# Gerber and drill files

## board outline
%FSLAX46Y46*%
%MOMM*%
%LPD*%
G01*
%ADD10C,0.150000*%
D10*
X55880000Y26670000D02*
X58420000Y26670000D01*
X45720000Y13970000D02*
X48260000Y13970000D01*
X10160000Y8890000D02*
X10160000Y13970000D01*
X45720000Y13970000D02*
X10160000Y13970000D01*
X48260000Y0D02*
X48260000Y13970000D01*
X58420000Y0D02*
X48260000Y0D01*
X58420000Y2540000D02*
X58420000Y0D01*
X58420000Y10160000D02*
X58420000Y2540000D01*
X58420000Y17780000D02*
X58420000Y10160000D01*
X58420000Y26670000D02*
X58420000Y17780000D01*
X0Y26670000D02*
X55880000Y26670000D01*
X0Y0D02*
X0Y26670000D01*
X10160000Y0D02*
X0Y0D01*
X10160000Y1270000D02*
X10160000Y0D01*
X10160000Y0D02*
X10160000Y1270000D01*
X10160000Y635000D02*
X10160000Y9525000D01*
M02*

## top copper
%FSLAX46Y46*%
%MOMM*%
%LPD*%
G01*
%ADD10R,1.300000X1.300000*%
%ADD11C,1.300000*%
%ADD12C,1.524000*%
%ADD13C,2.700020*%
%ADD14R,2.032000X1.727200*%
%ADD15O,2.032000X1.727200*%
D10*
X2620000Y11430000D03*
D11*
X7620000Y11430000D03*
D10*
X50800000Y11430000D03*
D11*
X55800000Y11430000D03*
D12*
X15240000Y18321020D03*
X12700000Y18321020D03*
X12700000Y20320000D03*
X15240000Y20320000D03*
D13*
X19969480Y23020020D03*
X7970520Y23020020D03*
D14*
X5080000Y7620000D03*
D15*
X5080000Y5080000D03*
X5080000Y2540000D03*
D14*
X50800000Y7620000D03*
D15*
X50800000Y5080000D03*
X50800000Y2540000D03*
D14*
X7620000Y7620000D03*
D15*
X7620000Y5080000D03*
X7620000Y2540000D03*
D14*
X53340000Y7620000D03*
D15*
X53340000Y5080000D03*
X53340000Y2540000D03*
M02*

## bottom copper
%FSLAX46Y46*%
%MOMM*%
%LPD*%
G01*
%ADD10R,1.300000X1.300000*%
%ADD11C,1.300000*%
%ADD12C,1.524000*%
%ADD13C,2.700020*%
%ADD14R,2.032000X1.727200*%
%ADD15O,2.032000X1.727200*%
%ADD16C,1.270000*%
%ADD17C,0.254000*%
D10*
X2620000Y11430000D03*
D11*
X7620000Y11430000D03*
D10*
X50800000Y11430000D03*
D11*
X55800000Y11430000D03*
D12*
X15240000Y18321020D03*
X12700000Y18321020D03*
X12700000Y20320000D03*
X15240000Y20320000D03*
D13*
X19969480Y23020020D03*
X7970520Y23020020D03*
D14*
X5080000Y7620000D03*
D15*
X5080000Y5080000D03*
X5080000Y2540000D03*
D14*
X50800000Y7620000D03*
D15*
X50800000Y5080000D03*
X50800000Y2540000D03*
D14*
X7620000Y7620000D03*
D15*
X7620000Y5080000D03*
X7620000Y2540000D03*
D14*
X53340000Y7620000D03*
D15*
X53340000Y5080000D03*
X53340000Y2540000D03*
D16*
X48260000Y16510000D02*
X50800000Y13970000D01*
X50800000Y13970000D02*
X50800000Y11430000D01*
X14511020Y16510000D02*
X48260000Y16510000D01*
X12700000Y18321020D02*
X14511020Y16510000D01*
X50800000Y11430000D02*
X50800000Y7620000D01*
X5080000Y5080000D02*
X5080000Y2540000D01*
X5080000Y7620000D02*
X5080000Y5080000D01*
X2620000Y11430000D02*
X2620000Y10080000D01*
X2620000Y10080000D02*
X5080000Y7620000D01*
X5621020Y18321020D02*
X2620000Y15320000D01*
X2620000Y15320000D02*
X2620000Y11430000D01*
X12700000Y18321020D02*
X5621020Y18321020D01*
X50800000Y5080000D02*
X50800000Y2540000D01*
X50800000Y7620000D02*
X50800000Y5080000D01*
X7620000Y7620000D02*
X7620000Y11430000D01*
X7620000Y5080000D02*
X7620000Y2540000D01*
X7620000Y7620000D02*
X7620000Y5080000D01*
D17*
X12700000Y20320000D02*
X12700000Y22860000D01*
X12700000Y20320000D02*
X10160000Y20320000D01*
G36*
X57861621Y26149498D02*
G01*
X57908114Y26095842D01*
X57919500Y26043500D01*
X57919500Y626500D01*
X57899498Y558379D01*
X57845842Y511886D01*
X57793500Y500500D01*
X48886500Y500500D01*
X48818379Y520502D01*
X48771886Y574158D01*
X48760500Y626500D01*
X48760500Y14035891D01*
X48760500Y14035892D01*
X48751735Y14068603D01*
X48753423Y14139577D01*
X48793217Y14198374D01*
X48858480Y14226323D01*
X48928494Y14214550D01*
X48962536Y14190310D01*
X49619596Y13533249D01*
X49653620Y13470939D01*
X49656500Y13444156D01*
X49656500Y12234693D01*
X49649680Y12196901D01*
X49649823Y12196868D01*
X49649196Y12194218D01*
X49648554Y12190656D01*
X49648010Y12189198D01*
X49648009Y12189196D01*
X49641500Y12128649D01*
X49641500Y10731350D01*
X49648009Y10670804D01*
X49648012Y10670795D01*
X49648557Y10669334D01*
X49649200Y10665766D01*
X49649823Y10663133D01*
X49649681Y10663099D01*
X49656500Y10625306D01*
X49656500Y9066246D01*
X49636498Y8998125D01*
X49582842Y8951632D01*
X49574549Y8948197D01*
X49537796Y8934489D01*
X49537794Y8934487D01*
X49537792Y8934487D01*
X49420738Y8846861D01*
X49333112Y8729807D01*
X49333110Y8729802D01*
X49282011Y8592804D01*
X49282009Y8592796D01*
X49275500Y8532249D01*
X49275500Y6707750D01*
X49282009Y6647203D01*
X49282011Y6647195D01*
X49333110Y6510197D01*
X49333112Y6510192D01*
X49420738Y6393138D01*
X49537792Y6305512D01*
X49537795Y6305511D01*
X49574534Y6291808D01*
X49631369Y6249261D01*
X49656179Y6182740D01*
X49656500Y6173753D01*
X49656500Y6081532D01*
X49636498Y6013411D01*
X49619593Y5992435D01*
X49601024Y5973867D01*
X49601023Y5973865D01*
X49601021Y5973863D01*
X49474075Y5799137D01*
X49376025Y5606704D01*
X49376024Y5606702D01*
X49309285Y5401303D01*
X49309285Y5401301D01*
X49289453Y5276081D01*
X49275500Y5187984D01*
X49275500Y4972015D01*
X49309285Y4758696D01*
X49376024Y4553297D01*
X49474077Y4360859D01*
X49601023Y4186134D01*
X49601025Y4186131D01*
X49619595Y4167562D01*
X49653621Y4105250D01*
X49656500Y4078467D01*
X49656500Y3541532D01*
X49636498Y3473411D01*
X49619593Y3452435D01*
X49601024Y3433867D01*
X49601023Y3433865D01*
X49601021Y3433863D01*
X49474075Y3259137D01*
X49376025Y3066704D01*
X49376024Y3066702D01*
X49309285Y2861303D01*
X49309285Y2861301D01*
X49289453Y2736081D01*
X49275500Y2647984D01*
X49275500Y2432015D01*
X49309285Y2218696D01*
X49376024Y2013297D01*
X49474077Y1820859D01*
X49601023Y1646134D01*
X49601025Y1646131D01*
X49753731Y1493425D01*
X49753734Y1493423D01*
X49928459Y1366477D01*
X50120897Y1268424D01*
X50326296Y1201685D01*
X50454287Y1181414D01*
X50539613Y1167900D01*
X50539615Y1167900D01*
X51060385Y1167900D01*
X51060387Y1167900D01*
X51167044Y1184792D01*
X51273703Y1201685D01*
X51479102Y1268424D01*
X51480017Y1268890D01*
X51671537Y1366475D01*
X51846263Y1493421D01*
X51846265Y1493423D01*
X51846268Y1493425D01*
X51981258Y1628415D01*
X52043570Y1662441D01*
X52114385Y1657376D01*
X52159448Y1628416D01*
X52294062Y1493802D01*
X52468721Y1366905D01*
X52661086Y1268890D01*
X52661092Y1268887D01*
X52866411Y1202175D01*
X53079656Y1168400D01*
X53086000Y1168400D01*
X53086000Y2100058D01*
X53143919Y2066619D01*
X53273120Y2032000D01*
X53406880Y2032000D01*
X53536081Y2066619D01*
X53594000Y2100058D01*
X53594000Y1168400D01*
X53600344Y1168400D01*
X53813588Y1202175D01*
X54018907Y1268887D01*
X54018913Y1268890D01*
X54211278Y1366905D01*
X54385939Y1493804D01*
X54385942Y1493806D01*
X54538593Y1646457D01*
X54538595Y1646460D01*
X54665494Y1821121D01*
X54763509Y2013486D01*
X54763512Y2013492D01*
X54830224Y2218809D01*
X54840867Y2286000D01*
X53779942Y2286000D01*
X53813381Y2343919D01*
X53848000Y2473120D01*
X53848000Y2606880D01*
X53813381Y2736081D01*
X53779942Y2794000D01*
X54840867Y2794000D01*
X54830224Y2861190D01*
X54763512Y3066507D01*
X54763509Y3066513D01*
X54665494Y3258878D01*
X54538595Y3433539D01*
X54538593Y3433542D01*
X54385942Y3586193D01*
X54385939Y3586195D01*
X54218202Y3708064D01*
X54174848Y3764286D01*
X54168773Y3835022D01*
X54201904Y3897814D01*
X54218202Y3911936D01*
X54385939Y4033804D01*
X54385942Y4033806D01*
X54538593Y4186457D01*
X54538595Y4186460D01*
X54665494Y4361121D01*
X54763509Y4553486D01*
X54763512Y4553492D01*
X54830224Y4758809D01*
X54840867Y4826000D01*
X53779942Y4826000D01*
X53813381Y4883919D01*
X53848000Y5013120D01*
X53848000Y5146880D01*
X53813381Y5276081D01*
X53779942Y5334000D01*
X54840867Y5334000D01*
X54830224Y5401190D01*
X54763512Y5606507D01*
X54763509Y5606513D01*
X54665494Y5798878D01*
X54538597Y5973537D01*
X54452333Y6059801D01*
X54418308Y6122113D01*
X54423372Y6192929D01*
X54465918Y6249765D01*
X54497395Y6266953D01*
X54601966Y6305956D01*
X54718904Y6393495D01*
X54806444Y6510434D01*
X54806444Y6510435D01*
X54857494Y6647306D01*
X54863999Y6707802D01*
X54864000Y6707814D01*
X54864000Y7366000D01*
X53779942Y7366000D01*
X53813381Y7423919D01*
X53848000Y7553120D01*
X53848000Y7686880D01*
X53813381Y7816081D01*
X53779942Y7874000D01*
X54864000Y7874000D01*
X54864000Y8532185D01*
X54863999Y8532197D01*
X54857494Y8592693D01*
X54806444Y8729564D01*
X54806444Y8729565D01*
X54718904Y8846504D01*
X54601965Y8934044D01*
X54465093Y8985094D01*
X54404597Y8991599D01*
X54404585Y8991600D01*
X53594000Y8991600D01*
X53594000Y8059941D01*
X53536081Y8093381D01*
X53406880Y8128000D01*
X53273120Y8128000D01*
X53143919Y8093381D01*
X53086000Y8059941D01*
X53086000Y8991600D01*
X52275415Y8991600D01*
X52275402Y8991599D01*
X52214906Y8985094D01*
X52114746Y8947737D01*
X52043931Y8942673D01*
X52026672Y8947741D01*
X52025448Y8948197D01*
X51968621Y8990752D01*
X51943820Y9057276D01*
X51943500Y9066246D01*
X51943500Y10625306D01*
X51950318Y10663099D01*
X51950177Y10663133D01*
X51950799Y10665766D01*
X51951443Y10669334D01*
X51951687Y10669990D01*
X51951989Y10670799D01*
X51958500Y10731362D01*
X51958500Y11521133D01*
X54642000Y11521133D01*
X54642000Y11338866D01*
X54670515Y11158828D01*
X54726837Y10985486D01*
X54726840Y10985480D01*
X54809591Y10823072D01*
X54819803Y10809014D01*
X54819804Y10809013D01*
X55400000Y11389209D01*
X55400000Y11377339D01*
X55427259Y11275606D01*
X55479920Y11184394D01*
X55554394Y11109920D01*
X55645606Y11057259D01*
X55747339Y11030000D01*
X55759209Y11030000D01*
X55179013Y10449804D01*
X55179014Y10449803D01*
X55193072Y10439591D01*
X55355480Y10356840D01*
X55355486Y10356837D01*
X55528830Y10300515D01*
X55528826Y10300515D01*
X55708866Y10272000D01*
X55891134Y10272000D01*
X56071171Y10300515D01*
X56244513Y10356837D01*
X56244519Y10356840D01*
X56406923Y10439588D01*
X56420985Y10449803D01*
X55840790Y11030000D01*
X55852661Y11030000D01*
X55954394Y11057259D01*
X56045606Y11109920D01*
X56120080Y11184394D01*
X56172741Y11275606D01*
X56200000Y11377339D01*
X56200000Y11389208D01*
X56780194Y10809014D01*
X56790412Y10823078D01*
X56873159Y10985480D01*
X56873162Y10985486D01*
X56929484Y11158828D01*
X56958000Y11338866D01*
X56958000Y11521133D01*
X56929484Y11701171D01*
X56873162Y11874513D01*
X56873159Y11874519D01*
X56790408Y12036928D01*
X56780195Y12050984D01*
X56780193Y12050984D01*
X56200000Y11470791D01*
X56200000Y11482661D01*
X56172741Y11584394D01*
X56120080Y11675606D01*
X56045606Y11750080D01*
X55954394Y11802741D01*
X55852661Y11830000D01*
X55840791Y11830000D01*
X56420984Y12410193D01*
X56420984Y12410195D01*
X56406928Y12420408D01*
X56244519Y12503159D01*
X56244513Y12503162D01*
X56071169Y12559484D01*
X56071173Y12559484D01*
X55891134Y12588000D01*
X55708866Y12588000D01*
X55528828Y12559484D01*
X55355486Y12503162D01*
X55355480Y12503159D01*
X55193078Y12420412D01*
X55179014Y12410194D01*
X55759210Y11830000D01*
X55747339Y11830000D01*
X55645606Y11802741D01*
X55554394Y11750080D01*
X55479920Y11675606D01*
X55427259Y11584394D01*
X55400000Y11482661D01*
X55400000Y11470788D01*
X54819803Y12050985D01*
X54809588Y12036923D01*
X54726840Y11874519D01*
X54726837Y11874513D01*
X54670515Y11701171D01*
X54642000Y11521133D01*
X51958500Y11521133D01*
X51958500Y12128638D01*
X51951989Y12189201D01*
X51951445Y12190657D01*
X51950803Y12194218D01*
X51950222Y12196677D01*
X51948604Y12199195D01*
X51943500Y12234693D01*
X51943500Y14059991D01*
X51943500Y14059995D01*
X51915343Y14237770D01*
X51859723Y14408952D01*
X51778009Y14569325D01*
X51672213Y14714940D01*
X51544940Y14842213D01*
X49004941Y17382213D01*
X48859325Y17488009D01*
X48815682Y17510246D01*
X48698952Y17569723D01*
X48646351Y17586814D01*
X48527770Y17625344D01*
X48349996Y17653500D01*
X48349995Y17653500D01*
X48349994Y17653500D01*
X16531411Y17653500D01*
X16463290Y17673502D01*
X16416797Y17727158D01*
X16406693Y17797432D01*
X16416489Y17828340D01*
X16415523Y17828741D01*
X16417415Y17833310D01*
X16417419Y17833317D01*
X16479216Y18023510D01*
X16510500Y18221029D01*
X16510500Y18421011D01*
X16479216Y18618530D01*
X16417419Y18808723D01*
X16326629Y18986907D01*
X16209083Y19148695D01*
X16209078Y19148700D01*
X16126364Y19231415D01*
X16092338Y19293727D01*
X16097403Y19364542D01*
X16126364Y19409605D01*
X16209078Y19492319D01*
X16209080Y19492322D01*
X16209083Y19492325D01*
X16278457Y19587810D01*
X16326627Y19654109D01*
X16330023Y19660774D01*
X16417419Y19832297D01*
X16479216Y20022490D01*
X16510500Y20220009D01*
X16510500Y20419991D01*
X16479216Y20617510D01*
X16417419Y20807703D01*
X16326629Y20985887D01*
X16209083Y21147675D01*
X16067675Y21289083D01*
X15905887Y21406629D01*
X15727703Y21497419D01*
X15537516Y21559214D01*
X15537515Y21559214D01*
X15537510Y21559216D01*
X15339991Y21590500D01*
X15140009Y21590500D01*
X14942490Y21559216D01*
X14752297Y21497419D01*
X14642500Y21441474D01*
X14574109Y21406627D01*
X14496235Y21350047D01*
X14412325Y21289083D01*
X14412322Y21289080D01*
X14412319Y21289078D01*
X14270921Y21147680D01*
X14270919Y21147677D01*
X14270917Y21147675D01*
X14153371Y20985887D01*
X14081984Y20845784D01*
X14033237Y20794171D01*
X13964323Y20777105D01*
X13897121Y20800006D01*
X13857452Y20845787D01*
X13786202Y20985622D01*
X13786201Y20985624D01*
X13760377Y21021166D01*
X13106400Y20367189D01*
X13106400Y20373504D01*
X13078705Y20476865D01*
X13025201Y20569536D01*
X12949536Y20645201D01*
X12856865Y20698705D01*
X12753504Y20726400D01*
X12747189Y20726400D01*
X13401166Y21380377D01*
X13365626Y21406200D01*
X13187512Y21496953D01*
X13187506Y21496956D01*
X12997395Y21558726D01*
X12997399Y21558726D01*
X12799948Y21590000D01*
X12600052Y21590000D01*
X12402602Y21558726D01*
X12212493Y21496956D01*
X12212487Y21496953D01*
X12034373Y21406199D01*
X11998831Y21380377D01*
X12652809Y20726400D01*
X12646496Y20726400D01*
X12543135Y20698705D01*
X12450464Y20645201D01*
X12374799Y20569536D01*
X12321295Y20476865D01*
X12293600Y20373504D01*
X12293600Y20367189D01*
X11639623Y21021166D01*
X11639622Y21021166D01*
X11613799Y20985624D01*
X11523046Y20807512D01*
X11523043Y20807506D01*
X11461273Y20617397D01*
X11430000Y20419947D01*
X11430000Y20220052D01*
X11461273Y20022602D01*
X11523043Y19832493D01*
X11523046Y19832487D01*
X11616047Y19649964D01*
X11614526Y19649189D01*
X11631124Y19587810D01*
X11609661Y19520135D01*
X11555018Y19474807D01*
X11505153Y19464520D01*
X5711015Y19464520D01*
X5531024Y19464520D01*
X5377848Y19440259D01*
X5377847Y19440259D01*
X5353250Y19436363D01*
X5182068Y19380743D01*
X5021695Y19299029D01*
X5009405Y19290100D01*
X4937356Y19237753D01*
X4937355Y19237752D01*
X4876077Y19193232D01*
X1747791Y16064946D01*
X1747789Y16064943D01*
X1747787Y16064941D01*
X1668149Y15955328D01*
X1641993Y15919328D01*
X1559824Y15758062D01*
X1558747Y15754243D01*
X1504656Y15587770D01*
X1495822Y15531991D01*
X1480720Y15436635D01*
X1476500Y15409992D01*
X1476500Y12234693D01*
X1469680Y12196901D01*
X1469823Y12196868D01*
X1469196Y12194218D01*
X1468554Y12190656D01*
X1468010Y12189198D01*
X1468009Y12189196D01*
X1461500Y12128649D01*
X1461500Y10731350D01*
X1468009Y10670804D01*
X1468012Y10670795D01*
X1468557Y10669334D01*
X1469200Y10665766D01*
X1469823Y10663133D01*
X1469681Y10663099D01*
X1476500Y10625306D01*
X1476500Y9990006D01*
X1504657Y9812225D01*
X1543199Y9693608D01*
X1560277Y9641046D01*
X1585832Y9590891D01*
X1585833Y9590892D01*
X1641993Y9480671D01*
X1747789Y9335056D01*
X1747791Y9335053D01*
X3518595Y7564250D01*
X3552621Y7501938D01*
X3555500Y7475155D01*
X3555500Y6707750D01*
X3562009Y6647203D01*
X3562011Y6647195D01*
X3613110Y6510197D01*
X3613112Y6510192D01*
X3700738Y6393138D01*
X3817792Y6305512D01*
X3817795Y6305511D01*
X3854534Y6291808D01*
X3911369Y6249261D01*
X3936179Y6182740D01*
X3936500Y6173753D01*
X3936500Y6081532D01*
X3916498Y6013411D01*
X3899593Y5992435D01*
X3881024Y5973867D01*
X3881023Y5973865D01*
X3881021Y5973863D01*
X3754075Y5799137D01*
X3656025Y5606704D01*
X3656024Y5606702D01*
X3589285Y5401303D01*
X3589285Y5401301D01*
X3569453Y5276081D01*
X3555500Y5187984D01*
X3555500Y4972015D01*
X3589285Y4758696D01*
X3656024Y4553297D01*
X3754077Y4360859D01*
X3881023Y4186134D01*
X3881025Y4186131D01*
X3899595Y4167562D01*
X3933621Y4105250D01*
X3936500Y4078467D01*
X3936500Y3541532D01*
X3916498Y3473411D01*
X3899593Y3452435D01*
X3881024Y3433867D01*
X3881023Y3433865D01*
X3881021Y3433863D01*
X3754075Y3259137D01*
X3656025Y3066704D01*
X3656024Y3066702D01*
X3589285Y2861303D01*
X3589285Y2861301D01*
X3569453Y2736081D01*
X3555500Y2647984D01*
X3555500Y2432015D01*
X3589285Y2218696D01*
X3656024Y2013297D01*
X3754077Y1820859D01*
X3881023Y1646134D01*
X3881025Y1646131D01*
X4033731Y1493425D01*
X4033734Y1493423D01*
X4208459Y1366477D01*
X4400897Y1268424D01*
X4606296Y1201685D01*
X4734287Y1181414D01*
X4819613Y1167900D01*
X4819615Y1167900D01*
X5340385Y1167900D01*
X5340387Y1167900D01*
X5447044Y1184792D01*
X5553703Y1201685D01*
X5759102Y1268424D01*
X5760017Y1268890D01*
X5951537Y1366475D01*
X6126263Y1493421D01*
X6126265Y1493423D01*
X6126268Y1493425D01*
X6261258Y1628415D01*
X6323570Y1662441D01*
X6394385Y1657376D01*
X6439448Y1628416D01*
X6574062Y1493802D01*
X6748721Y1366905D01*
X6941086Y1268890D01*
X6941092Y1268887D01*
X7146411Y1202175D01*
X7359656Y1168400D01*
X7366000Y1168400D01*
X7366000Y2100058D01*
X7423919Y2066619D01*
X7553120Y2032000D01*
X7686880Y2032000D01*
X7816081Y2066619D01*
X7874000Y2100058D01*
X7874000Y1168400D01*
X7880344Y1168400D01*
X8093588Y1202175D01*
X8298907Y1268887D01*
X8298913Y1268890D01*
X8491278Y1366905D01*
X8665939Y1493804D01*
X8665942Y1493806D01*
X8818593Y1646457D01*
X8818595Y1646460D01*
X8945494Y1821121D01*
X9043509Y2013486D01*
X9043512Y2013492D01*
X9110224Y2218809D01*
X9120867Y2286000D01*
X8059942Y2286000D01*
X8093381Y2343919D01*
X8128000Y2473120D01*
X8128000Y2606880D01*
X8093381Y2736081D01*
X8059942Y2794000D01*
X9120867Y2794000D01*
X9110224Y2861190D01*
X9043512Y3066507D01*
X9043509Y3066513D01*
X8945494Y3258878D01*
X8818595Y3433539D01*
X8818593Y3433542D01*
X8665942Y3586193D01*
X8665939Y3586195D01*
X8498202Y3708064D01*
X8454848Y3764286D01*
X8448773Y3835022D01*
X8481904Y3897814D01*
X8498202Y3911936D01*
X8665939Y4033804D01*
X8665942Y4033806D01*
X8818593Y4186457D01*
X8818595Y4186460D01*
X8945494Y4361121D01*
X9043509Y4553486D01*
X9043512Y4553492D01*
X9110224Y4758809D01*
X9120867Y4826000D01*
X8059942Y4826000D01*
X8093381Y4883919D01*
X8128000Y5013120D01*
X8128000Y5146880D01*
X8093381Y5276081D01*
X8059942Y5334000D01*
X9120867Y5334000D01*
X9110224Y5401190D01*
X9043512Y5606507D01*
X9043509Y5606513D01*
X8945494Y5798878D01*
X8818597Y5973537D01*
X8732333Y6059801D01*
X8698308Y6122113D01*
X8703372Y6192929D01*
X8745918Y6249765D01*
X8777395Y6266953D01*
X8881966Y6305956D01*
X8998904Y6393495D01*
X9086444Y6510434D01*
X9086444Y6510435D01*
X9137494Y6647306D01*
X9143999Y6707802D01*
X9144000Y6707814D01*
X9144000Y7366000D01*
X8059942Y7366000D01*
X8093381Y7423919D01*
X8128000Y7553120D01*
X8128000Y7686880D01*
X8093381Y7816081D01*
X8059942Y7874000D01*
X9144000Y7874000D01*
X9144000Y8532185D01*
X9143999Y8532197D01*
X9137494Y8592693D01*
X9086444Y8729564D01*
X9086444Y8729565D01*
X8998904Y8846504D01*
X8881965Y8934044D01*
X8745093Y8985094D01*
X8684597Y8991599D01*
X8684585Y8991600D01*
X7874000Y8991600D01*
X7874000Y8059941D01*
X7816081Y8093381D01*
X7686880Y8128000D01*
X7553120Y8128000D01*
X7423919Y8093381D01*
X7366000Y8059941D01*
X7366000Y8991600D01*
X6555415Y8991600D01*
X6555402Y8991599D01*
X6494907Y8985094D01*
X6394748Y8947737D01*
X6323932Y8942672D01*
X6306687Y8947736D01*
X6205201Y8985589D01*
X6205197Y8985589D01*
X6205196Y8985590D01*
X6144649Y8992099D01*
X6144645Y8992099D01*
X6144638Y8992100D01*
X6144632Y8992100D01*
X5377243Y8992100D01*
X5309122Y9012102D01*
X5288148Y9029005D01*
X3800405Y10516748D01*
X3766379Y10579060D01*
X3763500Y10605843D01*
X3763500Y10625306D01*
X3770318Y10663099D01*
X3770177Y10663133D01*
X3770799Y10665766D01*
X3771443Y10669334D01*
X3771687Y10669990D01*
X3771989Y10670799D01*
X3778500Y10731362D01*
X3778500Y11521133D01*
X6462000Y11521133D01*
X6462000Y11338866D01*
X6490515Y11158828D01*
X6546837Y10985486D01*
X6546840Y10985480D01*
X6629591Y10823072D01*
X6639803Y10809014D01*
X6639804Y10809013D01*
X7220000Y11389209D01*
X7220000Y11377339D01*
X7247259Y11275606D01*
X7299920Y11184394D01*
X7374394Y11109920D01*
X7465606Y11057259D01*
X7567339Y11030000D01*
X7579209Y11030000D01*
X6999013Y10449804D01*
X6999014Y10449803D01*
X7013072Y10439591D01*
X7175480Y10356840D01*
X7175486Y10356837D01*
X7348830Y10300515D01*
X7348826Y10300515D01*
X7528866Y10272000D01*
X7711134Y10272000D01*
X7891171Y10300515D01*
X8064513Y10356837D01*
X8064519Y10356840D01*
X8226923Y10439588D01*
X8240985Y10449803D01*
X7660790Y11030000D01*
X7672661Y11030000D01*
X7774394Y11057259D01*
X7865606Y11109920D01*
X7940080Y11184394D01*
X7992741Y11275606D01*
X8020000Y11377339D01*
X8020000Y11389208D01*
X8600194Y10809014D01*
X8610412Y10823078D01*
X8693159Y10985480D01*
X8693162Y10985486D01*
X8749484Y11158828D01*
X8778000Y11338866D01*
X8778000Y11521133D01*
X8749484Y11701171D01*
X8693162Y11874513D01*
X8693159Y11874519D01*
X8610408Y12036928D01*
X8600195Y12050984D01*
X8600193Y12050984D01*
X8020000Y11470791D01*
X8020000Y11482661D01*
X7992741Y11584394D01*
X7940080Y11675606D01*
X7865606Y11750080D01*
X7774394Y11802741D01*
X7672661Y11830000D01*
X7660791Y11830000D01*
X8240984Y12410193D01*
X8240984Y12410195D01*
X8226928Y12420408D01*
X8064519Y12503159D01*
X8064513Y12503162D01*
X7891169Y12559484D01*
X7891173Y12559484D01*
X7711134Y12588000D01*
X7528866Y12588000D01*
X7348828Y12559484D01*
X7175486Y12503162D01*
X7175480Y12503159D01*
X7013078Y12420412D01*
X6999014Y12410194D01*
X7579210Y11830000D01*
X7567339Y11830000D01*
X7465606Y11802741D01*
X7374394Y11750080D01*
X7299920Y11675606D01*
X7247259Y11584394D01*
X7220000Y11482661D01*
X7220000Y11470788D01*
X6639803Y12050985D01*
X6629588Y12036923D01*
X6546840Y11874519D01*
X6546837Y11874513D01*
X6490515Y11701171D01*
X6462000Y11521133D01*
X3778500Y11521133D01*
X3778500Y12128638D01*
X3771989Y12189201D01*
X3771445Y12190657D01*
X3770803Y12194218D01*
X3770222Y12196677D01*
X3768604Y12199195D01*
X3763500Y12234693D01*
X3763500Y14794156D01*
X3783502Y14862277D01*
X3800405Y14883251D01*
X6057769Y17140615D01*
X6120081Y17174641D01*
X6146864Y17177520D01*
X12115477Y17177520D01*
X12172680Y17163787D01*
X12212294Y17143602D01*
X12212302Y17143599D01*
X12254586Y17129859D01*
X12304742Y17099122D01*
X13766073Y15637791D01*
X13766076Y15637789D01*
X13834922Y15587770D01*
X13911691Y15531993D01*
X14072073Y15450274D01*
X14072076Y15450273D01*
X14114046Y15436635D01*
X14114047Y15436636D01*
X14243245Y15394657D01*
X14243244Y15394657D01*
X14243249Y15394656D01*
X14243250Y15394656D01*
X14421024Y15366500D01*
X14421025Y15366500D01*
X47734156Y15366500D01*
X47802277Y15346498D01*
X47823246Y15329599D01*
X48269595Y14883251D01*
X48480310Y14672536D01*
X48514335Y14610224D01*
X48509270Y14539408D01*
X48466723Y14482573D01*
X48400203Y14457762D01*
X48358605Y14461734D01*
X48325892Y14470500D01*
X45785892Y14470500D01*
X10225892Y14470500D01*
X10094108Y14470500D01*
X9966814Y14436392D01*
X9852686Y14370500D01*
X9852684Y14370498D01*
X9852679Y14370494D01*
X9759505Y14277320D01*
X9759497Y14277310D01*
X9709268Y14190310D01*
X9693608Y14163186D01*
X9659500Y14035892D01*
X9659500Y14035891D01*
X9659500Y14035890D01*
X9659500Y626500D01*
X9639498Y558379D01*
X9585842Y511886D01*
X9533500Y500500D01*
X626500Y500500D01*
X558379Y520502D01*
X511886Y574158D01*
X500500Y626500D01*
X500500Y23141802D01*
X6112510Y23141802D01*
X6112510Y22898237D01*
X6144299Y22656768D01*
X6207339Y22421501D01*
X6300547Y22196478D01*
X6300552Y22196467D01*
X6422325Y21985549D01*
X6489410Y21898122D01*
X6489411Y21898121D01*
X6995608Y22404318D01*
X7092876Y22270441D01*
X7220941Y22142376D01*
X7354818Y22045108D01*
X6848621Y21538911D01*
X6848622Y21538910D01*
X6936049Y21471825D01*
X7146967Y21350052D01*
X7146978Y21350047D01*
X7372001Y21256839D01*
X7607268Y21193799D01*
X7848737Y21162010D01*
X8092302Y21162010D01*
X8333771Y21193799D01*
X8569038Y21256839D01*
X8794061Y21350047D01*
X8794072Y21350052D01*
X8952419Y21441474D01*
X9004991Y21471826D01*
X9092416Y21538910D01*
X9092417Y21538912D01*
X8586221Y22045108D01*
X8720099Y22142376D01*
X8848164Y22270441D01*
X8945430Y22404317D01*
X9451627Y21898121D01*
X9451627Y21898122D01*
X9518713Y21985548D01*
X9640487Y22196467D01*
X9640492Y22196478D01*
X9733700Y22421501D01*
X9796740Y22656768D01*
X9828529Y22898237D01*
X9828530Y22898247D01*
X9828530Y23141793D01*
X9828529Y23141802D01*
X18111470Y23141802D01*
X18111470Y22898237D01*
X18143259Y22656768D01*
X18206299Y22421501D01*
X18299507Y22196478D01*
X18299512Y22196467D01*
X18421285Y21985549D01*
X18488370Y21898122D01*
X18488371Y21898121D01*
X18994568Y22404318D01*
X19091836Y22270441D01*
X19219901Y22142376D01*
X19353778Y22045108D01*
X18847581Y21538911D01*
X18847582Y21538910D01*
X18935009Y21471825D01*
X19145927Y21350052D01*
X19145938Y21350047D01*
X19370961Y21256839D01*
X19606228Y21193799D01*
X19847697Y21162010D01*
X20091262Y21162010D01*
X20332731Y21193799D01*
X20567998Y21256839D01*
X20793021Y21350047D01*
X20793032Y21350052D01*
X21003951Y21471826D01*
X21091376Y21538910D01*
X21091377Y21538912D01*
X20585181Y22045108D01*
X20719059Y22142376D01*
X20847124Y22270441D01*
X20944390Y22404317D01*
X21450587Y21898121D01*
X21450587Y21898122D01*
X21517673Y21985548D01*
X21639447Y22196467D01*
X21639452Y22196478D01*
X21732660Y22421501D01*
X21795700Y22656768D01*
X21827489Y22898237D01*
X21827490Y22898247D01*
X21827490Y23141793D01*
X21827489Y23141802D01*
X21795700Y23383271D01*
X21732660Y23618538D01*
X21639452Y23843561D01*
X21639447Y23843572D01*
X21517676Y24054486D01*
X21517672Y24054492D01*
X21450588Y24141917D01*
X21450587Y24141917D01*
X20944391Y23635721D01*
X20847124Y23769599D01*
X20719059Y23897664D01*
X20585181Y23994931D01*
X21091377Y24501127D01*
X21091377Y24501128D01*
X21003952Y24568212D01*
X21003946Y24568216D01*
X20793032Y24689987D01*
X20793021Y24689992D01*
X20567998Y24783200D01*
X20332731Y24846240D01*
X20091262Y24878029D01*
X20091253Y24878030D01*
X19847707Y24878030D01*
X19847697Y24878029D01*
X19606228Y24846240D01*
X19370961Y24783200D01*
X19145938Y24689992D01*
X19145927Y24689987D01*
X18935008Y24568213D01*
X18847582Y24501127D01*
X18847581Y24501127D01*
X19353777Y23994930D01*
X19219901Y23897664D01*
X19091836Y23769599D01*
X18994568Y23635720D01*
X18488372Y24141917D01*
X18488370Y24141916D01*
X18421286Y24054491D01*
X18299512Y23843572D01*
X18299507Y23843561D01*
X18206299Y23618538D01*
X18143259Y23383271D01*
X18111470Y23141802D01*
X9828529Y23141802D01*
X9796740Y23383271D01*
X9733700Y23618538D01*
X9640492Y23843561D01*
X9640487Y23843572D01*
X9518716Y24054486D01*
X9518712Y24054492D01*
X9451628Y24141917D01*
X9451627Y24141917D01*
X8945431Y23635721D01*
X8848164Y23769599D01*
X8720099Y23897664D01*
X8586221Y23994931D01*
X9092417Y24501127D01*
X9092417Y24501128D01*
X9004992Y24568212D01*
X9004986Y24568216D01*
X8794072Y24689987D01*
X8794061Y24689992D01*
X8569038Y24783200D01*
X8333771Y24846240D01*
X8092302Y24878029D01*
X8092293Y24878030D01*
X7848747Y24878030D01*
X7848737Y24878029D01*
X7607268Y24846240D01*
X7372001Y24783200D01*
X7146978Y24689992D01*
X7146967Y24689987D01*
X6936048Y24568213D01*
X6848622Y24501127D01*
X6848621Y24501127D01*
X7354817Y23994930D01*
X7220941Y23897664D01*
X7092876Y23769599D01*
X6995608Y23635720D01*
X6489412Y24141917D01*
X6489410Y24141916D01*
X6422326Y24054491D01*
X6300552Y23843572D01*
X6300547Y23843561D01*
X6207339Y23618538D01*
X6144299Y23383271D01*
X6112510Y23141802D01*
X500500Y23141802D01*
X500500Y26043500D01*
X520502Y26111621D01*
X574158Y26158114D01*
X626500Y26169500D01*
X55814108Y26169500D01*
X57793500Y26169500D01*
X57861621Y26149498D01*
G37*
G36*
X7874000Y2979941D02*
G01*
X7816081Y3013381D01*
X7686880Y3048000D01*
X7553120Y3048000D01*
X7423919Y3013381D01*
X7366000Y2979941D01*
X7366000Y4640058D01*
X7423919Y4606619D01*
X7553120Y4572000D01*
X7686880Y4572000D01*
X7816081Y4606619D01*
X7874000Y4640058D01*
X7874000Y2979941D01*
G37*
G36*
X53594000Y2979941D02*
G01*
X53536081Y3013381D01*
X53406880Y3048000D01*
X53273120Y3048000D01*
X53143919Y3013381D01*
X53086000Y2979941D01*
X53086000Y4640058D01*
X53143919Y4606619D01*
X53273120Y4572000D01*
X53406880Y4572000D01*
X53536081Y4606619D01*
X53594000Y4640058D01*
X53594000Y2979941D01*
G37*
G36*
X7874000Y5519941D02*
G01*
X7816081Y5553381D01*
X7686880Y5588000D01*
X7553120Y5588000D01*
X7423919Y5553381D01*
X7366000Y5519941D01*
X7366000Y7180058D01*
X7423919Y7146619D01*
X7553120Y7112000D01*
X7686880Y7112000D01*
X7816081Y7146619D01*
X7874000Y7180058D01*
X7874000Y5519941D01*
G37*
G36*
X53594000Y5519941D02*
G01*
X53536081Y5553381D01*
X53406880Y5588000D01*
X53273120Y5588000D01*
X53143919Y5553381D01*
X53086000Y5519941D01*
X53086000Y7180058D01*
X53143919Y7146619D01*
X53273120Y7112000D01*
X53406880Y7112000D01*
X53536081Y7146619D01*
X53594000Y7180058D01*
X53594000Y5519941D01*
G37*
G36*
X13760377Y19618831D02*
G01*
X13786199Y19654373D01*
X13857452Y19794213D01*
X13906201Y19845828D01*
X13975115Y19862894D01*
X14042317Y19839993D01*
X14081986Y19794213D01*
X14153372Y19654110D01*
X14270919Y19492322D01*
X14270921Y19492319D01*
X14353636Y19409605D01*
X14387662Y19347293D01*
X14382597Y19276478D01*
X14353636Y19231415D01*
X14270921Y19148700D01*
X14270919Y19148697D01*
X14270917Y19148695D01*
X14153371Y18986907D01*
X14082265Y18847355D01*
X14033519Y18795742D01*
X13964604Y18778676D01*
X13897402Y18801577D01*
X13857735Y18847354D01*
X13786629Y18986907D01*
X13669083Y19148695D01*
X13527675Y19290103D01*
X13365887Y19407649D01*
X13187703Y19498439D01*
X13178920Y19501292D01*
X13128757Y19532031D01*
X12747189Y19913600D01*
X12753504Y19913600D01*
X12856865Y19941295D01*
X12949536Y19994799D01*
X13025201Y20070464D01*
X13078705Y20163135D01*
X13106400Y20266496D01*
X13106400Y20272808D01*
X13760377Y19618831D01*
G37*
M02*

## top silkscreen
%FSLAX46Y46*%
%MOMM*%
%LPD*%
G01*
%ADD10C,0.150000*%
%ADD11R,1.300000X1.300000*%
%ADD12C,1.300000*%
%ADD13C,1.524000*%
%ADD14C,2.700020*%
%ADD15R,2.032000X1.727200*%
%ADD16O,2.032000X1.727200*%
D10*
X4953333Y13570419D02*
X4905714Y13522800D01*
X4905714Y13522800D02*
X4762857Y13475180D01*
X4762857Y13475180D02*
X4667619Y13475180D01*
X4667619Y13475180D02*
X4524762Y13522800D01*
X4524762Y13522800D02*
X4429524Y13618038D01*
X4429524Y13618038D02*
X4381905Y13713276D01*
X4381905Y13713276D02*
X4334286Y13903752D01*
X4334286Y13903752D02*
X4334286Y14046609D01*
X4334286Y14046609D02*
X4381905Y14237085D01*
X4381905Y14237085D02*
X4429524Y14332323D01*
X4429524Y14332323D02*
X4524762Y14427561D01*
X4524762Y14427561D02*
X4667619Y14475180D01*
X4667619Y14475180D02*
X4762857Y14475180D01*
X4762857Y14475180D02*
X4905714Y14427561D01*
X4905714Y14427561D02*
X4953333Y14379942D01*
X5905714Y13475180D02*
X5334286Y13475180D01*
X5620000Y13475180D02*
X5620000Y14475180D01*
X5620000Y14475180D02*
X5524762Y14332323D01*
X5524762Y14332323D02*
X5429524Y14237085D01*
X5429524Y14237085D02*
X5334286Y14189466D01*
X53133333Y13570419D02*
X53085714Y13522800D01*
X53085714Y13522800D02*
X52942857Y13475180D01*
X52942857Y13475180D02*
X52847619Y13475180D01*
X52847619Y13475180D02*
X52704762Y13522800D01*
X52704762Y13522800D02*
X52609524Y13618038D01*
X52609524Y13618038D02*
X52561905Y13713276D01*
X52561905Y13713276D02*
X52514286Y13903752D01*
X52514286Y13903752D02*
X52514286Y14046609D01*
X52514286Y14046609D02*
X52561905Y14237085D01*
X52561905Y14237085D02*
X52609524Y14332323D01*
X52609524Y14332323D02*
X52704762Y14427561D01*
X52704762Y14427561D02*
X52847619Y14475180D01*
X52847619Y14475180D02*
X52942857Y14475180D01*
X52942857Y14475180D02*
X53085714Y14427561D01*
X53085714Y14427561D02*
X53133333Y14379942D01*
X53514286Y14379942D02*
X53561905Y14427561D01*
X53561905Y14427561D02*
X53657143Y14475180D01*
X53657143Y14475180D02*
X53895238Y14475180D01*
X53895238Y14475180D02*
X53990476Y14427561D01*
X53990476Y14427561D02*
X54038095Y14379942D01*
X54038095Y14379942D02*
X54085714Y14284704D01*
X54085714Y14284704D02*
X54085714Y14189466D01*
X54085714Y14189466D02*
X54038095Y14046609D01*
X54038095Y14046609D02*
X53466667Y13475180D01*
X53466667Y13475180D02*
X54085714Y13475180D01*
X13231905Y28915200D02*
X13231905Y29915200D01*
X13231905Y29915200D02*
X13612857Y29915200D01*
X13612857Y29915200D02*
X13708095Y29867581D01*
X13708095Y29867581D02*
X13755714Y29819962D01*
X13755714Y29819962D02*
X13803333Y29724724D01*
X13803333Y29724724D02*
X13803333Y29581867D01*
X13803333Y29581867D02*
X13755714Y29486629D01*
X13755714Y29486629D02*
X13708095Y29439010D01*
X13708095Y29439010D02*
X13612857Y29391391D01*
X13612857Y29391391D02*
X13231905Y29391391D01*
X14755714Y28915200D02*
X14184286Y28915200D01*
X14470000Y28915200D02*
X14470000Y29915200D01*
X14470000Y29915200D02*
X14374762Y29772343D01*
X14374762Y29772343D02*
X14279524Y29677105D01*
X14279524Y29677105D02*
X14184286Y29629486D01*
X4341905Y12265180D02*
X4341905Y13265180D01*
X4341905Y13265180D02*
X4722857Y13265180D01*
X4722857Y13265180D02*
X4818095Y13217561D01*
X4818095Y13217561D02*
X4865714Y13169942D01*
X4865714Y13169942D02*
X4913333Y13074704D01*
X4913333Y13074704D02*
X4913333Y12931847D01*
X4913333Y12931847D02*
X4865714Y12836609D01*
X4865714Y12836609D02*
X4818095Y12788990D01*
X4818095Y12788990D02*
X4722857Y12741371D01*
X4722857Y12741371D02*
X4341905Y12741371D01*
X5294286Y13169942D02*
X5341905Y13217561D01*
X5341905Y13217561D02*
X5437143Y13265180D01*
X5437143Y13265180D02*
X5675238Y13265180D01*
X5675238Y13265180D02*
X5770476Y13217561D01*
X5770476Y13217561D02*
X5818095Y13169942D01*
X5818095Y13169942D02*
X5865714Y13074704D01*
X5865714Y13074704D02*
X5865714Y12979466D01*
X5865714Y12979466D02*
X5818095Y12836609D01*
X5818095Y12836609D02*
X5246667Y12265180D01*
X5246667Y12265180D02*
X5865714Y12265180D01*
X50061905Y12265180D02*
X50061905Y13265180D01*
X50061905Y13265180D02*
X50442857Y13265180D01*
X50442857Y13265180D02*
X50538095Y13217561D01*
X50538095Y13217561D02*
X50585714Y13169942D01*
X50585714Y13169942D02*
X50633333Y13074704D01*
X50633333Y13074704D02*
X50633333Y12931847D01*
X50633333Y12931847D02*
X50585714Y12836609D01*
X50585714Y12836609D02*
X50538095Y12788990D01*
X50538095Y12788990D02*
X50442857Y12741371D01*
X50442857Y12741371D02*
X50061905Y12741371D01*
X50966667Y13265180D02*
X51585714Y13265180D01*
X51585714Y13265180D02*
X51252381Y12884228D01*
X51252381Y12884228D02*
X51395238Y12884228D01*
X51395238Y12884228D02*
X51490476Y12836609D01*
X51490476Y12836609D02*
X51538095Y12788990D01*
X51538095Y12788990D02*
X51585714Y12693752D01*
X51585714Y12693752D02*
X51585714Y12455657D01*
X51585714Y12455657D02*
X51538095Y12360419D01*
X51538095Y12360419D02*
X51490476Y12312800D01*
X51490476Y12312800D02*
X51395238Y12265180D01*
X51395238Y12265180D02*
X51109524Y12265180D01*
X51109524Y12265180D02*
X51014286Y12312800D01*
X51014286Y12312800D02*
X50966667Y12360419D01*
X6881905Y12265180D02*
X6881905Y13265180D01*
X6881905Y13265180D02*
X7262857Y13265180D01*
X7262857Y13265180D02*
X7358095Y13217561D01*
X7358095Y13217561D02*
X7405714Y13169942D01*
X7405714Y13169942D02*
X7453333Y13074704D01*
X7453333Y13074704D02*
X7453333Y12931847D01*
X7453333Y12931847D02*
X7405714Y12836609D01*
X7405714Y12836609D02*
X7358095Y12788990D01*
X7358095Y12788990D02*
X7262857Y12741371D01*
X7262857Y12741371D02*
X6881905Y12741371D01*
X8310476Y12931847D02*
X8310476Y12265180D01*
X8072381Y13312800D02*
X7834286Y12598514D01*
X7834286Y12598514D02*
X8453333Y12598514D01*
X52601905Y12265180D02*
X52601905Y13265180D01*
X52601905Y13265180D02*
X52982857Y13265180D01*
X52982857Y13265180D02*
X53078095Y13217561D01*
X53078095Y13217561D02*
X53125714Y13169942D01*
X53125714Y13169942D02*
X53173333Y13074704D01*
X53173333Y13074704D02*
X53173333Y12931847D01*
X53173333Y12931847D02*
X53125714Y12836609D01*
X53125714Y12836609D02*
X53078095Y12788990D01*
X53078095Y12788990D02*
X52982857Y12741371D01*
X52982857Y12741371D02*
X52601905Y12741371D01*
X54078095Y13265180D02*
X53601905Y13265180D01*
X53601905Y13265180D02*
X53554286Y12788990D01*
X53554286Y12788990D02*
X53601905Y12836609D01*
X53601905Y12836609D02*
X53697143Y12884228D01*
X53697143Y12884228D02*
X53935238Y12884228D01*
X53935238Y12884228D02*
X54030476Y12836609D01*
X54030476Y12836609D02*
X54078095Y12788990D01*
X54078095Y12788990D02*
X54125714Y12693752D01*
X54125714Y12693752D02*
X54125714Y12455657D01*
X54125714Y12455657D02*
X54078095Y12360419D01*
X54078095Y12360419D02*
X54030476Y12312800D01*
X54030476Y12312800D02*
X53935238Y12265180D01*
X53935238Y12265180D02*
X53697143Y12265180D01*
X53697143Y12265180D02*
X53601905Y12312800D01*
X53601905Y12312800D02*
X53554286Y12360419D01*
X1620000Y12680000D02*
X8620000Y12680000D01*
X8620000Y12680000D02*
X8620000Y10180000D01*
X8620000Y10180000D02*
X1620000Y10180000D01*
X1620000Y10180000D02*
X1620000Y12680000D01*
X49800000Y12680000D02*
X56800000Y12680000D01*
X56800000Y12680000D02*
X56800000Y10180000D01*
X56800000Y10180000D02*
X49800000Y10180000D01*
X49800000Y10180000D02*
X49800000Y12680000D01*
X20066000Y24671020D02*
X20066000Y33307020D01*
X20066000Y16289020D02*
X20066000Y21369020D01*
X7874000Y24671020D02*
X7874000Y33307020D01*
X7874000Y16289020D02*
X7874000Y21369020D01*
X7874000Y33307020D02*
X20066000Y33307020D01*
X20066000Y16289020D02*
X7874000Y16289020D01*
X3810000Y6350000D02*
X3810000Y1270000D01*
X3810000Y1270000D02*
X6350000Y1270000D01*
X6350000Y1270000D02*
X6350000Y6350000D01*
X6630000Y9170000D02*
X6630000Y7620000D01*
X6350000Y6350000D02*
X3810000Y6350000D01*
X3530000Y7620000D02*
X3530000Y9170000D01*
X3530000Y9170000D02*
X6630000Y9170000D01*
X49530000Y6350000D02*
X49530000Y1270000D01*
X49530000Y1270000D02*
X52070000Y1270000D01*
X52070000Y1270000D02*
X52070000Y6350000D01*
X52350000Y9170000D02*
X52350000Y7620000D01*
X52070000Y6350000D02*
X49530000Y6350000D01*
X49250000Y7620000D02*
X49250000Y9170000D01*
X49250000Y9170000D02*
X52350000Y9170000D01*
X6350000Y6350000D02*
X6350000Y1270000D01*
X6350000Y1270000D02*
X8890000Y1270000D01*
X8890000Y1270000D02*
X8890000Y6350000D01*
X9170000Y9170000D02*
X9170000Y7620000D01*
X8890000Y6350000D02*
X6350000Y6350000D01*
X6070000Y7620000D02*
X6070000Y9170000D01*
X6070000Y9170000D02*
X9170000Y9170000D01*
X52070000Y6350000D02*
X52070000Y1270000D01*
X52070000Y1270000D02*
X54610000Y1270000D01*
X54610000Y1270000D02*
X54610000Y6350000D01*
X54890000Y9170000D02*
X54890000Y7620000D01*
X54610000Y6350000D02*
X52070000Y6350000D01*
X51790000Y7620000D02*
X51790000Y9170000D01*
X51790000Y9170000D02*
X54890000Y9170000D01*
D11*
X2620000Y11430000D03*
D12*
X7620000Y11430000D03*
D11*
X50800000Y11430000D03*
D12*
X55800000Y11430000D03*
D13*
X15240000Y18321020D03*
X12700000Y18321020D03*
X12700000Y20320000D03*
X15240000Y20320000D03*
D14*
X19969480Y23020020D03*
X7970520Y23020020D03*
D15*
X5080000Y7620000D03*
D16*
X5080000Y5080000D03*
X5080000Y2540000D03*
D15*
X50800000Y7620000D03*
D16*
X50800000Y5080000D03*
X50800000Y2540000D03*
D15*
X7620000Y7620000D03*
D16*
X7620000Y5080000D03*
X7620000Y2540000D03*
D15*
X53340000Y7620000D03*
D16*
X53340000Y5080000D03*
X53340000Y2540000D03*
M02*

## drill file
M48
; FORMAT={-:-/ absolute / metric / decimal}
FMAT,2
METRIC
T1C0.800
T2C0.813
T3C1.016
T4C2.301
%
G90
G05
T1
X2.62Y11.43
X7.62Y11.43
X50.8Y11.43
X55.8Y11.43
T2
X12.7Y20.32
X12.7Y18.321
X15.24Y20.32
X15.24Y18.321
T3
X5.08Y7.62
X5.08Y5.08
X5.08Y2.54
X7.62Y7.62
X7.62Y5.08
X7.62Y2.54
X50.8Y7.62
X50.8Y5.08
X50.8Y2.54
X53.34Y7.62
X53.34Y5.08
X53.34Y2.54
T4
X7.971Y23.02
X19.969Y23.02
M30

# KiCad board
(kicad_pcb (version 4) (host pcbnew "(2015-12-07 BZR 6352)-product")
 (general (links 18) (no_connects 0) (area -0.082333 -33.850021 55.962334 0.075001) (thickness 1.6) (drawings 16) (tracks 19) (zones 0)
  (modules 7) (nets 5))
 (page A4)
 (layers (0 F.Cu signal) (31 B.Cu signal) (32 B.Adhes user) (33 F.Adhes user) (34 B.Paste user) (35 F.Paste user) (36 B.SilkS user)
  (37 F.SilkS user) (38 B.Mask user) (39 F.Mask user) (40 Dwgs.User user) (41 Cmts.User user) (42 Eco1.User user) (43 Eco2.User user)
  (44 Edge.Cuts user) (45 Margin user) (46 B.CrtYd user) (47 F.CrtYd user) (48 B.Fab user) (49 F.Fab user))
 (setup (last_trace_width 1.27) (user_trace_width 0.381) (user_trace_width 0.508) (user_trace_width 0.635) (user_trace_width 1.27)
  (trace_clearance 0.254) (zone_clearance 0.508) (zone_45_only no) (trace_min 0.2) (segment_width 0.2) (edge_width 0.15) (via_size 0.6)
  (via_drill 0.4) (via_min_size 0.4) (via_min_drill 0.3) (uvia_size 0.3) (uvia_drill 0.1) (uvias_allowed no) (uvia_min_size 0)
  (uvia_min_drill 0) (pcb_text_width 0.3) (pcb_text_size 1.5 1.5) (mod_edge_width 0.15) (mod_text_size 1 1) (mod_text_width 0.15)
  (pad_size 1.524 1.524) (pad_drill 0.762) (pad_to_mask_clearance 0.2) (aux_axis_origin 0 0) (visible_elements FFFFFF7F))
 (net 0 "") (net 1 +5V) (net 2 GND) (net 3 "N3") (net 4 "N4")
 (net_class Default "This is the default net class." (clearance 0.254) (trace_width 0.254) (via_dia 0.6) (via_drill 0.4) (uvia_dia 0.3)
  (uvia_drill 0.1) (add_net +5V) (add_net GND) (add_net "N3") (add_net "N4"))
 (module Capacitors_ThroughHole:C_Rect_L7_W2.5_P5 (layer F.Cu) (at 2.62 -11.43)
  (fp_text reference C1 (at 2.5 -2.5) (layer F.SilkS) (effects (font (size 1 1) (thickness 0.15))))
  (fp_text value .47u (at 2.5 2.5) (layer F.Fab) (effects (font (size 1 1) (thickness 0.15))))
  (fp_line (start -1 -1.25) (end 6 -1.25) (layer F.SilkS) (width 0.15))
  (fp_line (start 6 -1.25) (end 6 1.25) (layer F.SilkS) (width 0.15))
  (fp_line (start 6 1.25) (end -1 1.25) (layer F.SilkS) (width 0.15))
  (fp_line (start -1 1.25) (end -1 -1.25) (layer F.SilkS) (width 0.15))
  (pad 1 thru_hole rect (at 0 0) (size 1.3 1.3) (drill 0.8) (layers *.Cu *.Mask F.SilkS) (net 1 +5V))
  (pad 2 thru_hole circle (at 5 0) (size 1.3 1.3) (drill 0.8) (layers *.Cu *.Mask F.SilkS) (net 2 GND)))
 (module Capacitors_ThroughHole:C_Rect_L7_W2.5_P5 (layer F.Cu) (at 50.8 -11.43)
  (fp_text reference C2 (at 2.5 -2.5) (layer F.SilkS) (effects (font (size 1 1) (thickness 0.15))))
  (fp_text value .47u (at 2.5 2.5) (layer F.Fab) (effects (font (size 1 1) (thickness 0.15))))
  (fp_line (start -1 -1.25) (end 6 -1.25) (layer F.SilkS) (width 0.15))
  (fp_line (start 6 -1.25) (end 6 1.25) (layer F.SilkS) (width 0.15))
  (fp_line (start 6 1.25) (end -1 1.25) (layer F.SilkS) (width 0.15))
  (fp_line (start -1 1.25) (end -1 -1.25) (layer F.SilkS) (width 0.15))
  (pad 1 thru_hole rect (at 0 0) (size 1.3 1.3) (drill 0.8) (layers *.Cu *.Mask F.SilkS) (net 1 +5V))
  (pad 2 thru_hole circle (at 5 0) (size 1.3 1.3) (drill 0.8) (layers *.Cu *.Mask F.SilkS) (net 2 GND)))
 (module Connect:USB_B (layer F.Cu) (at 12.7 -18.32102 90)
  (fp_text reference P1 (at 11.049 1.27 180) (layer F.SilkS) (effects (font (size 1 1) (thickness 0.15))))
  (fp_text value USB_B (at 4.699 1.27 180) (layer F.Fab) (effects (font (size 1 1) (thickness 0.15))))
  (fp_line (start 6.35 7.366) (end 14.986 7.366) (layer F.SilkS) (width 0.15))
  (fp_line (start -2.032 7.366) (end 3.048 7.366) (layer F.SilkS) (width 0.15))
  (fp_line (start 6.35 -4.826) (end 14.986 -4.826) (layer F.SilkS) (width 0.15))
  (fp_line (start -2.032 -4.826) (end 3.048 -4.826) (layer F.SilkS) (width 0.15))
  (fp_line (start 14.986 -4.826) (end 14.986 7.366) (layer F.SilkS) (width 0.15))
  (fp_line (start -2.032 7.366) (end -2.032 -4.826) (layer F.SilkS) (width 0.15))
  (pad 2 thru_hole circle (at 0 2.54) (size 1.524 1.524) (drill 0.8128) (layers *.Cu *.Mask F.SilkS) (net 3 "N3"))
  (pad 1 thru_hole circle (at 0 0) (size 1.524 1.524) (drill 0.8128) (layers *.Cu *.Mask F.SilkS) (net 1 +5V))
  (pad 4 thru_hole circle (at 1.99898 0) (size 1.524 1.524) (drill 0.8128) (layers *.Cu *.Mask F.SilkS) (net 2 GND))
  (pad 3 thru_hole circle (at 1.99898 2.54) (size 1.524 1.524) (drill 0.8128) (layers *.Cu *.Mask F.SilkS) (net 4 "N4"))
  (pad 5 thru_hole circle (at 4.699 7.26948) (size 2.70002 2.70002) (drill 2.30124) (layers *.Cu *.Mask F.SilkS) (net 2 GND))
  (pad 5 thru_hole circle (at 4.699 -4.72948) (size 2.70002 2.70002) (drill 2.30124) (layers *.Cu *.Mask F.SilkS) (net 2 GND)))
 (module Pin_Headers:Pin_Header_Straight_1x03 (layer F.Cu) (at 5.08 -7.62)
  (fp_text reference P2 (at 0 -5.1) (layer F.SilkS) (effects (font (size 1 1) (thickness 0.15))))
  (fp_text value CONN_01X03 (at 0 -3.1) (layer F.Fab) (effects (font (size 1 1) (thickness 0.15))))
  (fp_line (start -1.27 1.27) (end -1.27 6.35) (layer F.SilkS) (width 0.15))
  (fp_line (start -1.27 6.35) (end 1.27 6.35) (layer F.SilkS) (width 0.15))
  (fp_line (start 1.27 6.35) (end 1.27 1.27) (layer F.SilkS) (width 0.15))
  (fp_line (start 1.55 -1.55) (end 1.55 0) (layer F.SilkS) (width 0.15))
  (fp_line (start 1.27 1.27) (end -1.27 1.27) (layer F.SilkS) (width 0.15))
  (fp_line (start -1.55 0) (end -1.55 -1.55) (layer F.SilkS) (width 0.15))
  (fp_line (start -1.55 -1.55) (end 1.55 -1.55) (layer F.SilkS) (width 0.15))
  (pad 1 thru_hole rect (at 0 0) (size 2.032 1.7272) (drill 1.016) (layers *.Cu *.Mask F.SilkS) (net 1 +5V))
  (pad 2 thru_hole oval (at 0 2.54) (size 2.032 1.7272) (drill 1.016) (layers *.Cu *.Mask F.SilkS) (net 1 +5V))
  (pad 3 thru_hole oval (at 0 5.08) (size 2.032 1.7272) (drill 1.016) (layers *.Cu *.Mask F.SilkS) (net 1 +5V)))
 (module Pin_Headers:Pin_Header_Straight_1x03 (layer F.Cu) (at 50.8 -7.62)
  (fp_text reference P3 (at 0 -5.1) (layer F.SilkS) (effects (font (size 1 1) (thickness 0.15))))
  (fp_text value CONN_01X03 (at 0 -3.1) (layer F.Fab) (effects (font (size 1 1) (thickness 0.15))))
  (fp_line (start -1.27 1.27) (end -1.27 6.35) (layer F.SilkS) (width 0.15))
  (fp_line (start -1.27 6.35) (end 1.27 6.35) (layer F.SilkS) (width 0.15))
  (fp_line (start 1.27 6.35) (end 1.27 1.27) (layer F.SilkS) (width 0.15))
  (fp_line (start 1.55 -1.55) (end 1.55 0) (layer F.SilkS) (width 0.15))
  (fp_line (start 1.27 1.27) (end -1.27 1.27) (layer F.SilkS) (width 0.15))
  (fp_line (start -1.55 0) (end -1.55 -1.55) (layer F.SilkS) (width 0.15))
  (fp_line (start -1.55 -1.55) (end 1.55 -1.55) (layer F.SilkS) (width 0.15))
  (pad 1 thru_hole rect (at 0 0) (size 2.032 1.7272) (drill 1.016) (layers *.Cu *.Mask F.SilkS) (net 1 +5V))
  (pad 2 thru_hole oval (at 0 2.54) (size 2.032 1.7272) (drill 1.016) (layers *.Cu *.Mask F.SilkS) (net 1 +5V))
  (pad 3 thru_hole oval (at 0 5.08) (size 2.032 1.7272) (drill 1.016) (layers *.Cu *.Mask F.SilkS) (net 1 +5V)))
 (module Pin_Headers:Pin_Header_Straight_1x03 (layer F.Cu) (at 7.62 -7.62)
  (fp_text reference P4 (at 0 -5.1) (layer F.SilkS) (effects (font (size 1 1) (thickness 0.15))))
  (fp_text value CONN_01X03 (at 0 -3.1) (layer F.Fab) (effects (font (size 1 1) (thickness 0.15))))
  (fp_line (start -1.27 1.27) (end -1.27 6.35) (layer F.SilkS) (width 0.15))
  (fp_line (start -1.27 6.35) (end 1.27 6.35) (layer F.SilkS) (width 0.15))
  (fp_line (start 1.27 6.35) (end 1.27 1.27) (layer F.SilkS) (width 0.15))
  (fp_line (start 1.55 -1.55) (end 1.55 0) (layer F.SilkS) (width 0.15))
  (fp_line (start 1.27 1.27) (end -1.27 1.27) (layer F.SilkS) (width 0.15))
  (fp_line (start -1.55 0) (end -1.55 -1.55) (layer F.SilkS) (width 0.15))
  (fp_line (start -1.55 -1.55) (end 1.55 -1.55) (layer F.SilkS) (width 0.15))
  (pad 1 thru_hole rect (at 0 0) (size 2.032 1.7272) (drill 1.016) (layers *.Cu *.Mask F.SilkS) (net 2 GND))
  (pad 2 thru_hole oval (at 0 2.54) (size 2.032 1.7272) (drill 1.016) (layers *.Cu *.Mask F.SilkS) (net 2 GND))
  (pad 3 thru_hole oval (at 0 5.08) (size 2.032 1.7272) (drill 1.016) (layers *.Cu *.Mask F.SilkS) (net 2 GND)))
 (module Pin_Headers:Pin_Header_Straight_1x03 (layer F.Cu) (at 53.34 -7.62)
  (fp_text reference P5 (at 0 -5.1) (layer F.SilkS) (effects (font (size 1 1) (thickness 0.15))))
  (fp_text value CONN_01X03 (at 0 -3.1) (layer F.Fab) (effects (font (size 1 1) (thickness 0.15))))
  (fp_line (start -1.27 1.27) (end -1.27 6.35) (layer F.SilkS) (width 0.15))
  (fp_line (start -1.27 6.35) (end 1.27 6.35) (layer F.SilkS) (width 0.15))
  (fp_line (start 1.27 6.35) (end 1.27 1.27) (layer F.SilkS) (width 0.15))
  (fp_line (start 1.55 -1.55) (end 1.55 0) (layer F.SilkS) (width 0.15))
  (fp_line (start 1.27 1.27) (end -1.27 1.27) (layer F.SilkS) (width 0.15))
  (fp_line (start -1.55 0) (end -1.55 -1.55) (layer F.SilkS) (width 0.15))
  (fp_line (start -1.55 -1.55) (end 1.55 -1.55) (layer F.SilkS) (width 0.15))
  (pad 1 thru_hole rect (at 0 0) (size 2.032 1.7272) (drill 1.016) (layers *.Cu *.Mask F.SilkS) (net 2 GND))
  (pad 2 thru_hole oval (at 0 2.54) (size 2.032 1.7272) (drill 1.016) (layers *.Cu *.Mask F.SilkS) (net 2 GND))
  (pad 3 thru_hole oval (at 0 5.08) (size 2.032 1.7272) (drill 1.016) (layers *.Cu *.Mask F.SilkS) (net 2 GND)))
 (gr_line (start 55.88 -26.67) (end 58.42 -26.67) (layer Edge.Cuts) (width 0.15))
 (gr_line (start 45.72 -13.97) (end 48.26 -13.97) (layer Edge.Cuts) (width 0.15))
 (gr_line (start 10.16 -8.89) (end 10.16 -13.97) (layer Edge.Cuts) (width 0.15))
 (gr_line (start 45.72 -13.97) (end 10.16 -13.97) (layer Edge.Cuts) (width 0.15))
 (gr_line (start 48.26 0) (end 48.26 -13.97) (layer Edge.Cuts) (width 0.15))
 (gr_line (start 58.42 0) (end 48.26 0) (layer Edge.Cuts) (width 0.15))
 (gr_line (start 58.42 -2.54) (end 58.42 0) (layer Edge.Cuts) (width 0.15))
 (gr_line (start 58.42 -10.16) (end 58.42 -2.54) (layer Edge.Cuts) (width 0.15))
 (gr_line (start 58.42 -17.78) (end 58.42 -10.16) (layer Edge.Cuts) (width 0.15))
 (gr_line (start 58.42 -26.67) (end 58.42 -17.78) (layer Edge.Cuts) (width 0.15))
 (gr_line (start 0 -26.67) (end 55.88 -26.67) (layer Edge.Cuts) (width 0.15))
 (gr_line (start 0 0) (end 0 -26.67) (layer Edge.Cuts) (width 0.15))
 (gr_line (start 10.16 0) (end 0 0) (layer Edge.Cuts) (width 0.15))
 (gr_line (start 10.16 -1.27) (end 10.16 0) (layer Edge.Cuts) (width 0.15))
 (gr_line (start 10.16 0) (end 10.16 -1.27) (layer Edge.Cuts) (width 0.15))
 (gr_line (start 10.16 -0.635) (end 10.16 -9.525) (layer Edge.Cuts) (width 0.15))
 (segment (start 48.26 -16.51) (end 50.8 -13.97) (width 1.27) (layer B.Cu) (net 1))
 (segment (start 50.8 -13.97) (end 50.8 -11.43) (width 1.27) (layer B.Cu) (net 1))
 (segment (start 14.51102 -16.51) (end 48.26 -16.51) (width 1.27) (layer B.Cu) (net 1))
 (segment (start 12.7 -18.32102) (end 14.51102 -16.51) (width 1.27) (layer B.Cu) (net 1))
 (segment (start 50.8 -11.43) (end 50.8 -7.62) (width 1.27) (layer B.Cu) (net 1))
 (segment (start 5.08 -5.08) (end 5.08 -2.54) (width 1.27) (layer B.Cu) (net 1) (status 30))
 (segment (start 5.08 -7.62) (end 5.08 -5.08) (width 1.27) (layer B.Cu) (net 1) (status 30))
 (segment (start 2.62 -11.43) (end 2.62 -10.08) (width 1.27) (layer B.Cu) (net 1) (status 10))
 (segment (start 2.62 -10.08) (end 5.08 -7.62) (width 1.27) (layer B.Cu) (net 1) (status 20))
 (segment (start 5.62102 -18.32102) (end 2.62 -15.32) (width 1.27) (layer B.Cu) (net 1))
 (segment (start 2.62 -15.32) (end 2.62 -11.43) (width 1.27) (layer B.Cu) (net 1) (status 20))
 (segment (start 12.7 -18.32102) (end 5.62102 -18.32102) (width 1.27) (layer B.Cu) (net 1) (status 10))
 (segment (start 50.8 -5.08) (end 50.8 -2.54) (width 1.27) (layer B.Cu) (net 1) (status 30))
 (segment (start 50.8 -7.62) (end 50.8 -5.08) (width 1.27) (layer B.Cu) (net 1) (status 30))
 (segment (start 7.62 -7.62) (end 7.62 -11.43) (width 1.27) (layer B.Cu) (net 2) (status 30))
 (segment (start 7.62 -5.08) (end 7.62 -2.54) (width 1.27) (layer B.Cu) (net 2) (status 30))
 (segment (start 7.62 -7.62) (end 7.62 -5.08) (width 1.27) (layer B.Cu) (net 2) (status 30))
 (segment (start 12.7 -20.32) (end 12.7 -22.86) (width 0.254) (layer B.Cu) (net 2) (status 10))
 (segment (start 12.7 -20.32) (end 10.16 -20.32) (width 0.254) (layer B.Cu) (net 2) (status 10))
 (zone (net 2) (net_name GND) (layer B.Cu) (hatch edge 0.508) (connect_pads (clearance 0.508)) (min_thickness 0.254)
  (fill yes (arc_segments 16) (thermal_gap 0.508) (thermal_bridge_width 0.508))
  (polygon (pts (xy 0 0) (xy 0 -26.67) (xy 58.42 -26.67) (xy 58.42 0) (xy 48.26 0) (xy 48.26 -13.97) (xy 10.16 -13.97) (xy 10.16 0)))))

